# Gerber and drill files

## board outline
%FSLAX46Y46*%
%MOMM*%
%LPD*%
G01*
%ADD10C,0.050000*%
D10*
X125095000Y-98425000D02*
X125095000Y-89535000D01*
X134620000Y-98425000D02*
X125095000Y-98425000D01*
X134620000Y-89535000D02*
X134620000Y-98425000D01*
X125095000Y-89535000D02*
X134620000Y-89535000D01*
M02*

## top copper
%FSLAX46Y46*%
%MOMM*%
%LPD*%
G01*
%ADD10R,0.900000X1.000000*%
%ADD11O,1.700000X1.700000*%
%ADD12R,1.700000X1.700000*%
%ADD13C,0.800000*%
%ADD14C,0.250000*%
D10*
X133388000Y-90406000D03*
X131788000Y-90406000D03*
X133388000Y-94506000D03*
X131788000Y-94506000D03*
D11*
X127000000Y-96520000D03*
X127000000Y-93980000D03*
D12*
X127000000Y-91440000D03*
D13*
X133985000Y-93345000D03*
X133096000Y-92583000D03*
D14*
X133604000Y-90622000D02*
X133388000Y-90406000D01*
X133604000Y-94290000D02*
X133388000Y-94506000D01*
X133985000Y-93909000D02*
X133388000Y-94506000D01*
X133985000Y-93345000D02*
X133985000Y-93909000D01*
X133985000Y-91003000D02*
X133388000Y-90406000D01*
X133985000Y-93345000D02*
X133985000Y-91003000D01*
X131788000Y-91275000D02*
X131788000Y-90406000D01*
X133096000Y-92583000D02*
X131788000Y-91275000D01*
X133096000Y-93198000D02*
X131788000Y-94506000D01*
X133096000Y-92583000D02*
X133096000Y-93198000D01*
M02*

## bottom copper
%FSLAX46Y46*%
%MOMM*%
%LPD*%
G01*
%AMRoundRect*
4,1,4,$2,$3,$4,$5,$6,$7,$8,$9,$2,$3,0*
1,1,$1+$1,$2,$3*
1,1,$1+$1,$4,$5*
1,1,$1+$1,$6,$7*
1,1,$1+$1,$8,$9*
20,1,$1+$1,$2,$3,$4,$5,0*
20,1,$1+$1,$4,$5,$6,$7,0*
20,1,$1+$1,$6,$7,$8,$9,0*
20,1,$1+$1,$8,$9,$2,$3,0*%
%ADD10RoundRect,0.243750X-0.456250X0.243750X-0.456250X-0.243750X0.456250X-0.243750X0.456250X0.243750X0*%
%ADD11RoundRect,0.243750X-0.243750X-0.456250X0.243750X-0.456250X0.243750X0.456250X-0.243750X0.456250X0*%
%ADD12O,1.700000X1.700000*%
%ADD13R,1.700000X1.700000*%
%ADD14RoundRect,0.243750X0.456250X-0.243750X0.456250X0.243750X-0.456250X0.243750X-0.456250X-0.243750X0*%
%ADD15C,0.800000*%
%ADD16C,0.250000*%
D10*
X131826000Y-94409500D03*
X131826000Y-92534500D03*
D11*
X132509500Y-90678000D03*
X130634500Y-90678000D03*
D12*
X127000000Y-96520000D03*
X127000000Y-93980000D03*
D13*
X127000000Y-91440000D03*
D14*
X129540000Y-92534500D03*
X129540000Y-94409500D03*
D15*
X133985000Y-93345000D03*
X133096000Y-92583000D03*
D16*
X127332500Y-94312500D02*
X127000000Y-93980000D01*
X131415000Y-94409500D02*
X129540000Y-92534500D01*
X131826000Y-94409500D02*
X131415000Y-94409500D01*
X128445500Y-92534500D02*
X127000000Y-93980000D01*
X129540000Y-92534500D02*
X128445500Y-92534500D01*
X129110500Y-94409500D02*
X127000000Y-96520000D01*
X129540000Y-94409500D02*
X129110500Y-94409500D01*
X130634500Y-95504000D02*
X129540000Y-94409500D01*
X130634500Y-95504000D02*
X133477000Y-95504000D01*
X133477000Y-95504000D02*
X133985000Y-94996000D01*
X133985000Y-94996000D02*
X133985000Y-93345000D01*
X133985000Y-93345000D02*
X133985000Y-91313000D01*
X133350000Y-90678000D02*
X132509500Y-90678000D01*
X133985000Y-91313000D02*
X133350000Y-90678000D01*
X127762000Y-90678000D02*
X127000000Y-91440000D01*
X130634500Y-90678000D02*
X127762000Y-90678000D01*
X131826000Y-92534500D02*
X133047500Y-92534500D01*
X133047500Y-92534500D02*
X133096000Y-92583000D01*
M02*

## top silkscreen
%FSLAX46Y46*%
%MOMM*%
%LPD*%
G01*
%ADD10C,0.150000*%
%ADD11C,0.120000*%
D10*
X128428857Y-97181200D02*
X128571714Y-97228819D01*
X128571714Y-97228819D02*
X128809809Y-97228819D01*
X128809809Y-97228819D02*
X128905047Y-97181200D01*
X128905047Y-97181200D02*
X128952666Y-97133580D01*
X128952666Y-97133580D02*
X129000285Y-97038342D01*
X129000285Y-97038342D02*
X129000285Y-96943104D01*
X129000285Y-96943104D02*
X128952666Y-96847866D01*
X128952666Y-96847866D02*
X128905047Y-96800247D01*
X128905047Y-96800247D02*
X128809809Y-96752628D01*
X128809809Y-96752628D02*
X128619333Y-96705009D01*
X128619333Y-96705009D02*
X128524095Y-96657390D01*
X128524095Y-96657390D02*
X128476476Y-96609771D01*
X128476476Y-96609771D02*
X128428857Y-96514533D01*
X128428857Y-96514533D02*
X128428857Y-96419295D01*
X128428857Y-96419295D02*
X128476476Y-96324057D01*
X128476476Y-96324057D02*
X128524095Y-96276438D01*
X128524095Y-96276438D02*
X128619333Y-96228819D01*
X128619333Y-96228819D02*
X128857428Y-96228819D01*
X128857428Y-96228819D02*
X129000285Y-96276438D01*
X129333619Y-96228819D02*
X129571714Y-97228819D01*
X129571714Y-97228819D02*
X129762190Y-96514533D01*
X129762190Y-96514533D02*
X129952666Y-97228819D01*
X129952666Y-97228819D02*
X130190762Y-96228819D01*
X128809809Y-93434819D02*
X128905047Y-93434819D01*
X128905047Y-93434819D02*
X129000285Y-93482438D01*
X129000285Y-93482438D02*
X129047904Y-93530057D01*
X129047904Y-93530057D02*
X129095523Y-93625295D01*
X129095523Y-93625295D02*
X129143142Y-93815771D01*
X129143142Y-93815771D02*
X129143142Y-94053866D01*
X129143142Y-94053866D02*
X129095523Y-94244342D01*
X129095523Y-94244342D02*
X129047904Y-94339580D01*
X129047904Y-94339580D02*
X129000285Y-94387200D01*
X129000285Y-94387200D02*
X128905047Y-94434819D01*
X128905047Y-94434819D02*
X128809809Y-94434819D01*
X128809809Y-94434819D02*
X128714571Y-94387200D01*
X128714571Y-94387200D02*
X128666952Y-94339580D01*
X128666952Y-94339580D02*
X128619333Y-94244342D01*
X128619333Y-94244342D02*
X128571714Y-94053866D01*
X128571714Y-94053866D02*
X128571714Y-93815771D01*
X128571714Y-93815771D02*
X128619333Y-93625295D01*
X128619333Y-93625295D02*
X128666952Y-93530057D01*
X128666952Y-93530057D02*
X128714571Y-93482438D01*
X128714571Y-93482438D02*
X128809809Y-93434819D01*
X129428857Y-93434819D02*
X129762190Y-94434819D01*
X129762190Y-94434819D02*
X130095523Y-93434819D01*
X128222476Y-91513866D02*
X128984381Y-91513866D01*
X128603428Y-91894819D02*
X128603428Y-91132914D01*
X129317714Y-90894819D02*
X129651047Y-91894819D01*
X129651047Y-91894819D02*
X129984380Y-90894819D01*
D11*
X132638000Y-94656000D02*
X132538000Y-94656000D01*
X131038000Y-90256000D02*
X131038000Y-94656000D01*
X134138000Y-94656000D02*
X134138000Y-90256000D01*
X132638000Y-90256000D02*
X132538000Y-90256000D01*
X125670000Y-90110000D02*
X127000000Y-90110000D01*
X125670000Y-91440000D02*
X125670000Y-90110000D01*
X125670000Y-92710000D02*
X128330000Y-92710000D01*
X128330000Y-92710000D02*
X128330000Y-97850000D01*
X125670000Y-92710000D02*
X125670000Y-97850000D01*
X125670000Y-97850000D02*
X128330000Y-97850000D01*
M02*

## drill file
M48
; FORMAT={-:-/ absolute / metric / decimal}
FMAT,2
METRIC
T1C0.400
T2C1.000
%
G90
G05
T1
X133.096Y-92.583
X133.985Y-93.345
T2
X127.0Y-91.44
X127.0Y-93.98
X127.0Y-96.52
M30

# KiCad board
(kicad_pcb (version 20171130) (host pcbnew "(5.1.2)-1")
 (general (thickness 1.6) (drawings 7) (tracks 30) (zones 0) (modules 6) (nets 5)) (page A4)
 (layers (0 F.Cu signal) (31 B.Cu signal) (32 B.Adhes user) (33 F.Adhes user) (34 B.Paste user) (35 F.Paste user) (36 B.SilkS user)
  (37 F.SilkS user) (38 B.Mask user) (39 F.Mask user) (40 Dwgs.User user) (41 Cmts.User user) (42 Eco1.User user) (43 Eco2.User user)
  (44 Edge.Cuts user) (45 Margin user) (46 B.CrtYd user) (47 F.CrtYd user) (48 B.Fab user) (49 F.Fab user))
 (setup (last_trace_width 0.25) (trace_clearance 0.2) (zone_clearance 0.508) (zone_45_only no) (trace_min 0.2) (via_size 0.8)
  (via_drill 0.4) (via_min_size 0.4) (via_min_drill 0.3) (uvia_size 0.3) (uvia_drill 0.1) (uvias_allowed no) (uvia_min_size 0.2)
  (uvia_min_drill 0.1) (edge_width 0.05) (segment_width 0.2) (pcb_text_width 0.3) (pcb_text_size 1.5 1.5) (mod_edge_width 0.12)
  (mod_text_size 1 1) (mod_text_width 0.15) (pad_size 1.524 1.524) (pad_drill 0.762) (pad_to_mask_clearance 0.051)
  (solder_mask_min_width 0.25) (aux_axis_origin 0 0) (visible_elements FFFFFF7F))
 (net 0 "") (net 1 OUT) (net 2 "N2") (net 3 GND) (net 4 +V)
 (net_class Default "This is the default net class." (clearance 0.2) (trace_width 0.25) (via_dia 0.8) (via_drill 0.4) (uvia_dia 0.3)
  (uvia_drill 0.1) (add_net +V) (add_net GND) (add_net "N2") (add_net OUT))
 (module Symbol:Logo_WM (layer B.Cu) (at 131.953 97.155)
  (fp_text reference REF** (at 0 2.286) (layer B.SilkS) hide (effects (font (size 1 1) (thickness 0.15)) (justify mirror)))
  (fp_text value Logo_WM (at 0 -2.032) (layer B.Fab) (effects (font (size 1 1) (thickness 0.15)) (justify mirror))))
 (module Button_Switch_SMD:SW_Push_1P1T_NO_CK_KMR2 (layer F.Cu) (at 132.588 92.456 90)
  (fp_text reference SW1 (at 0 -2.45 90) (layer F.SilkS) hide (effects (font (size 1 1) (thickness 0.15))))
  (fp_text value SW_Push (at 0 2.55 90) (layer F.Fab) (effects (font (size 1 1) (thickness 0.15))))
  (fp_line (start -2.2 0.05) (end -2.2 -0.05) (layer F.SilkS) (width 0.12))
  (fp_line (start 2.2 -1.55) (end -2.2 -1.55) (layer F.SilkS) (width 0.12))
  (fp_line (start -2.2 1.55) (end 2.2 1.55) (layer F.SilkS) (width 0.12))
  (fp_line (start 2.2 0.05) (end 2.2 -0.05) (layer F.SilkS) (width 0.12))
  (pad 2 smd rect (at 2.05 0.8 180) (size 0.9 1) (layers F.Cu F.Paste F.Mask) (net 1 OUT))
  (pad 1 smd rect (at 2.05 -0.8 180) (size 0.9 1) (layers F.Cu F.Paste F.Mask) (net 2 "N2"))
  (pad 2 smd rect (at -2.05 0.8 180) (size 0.9 1) (layers F.Cu F.Paste F.Mask) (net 1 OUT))
  (pad 1 smd rect (at -2.05 -0.8 180) (size 0.9 1) (layers F.Cu F.Paste F.Mask) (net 2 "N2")))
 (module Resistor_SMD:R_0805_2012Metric (layer B.Cu) (at 131.826 93.472 270)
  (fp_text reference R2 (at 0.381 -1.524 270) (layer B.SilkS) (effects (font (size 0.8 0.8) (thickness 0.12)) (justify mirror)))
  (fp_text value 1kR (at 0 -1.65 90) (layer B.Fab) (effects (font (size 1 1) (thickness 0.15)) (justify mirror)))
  (pad 2 smd roundrect (at 0.9375 0 270) (size 0.975 1.4) (layers B.Cu B.Paste B.Mask) (roundrect_rratio 0.25) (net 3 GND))
  (pad 1 smd roundrect (at -0.9375 0 270) (size 0.975 1.4) (layers B.Cu B.Paste B.Mask) (roundrect_rratio 0.25) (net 2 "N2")))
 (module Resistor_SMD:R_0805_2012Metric (layer B.Cu) (at 131.572 90.678)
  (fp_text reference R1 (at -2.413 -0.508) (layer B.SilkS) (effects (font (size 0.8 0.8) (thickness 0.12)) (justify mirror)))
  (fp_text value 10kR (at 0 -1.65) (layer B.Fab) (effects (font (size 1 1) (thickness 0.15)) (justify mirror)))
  (pad 2 smd roundrect (at 0.9375 0) (size 0.975 1.4) (layers B.Cu B.Paste B.Mask) (roundrect_rratio 0.25) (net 1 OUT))
  (pad 1 smd roundrect (at -0.9375 0) (size 0.975 1.4) (layers B.Cu B.Paste B.Mask) (roundrect_rratio 0.25) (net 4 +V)))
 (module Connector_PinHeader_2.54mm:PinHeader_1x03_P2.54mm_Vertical (layer F.Cu) (at 127 91.44)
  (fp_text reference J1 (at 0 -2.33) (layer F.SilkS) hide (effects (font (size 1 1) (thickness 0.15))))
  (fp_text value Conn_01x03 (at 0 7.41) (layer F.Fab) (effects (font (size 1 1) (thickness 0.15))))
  (fp_line (start -1.33 -1.33) (end 0 -1.33) (layer F.SilkS) (width 0.12))
  (fp_line (start -1.33 0) (end -1.33 -1.33) (layer F.SilkS) (width 0.12))
  (fp_line (start -1.33 1.27) (end 1.33 1.27) (layer F.SilkS) (width 0.12))
  (fp_line (start 1.33 1.27) (end 1.33 6.41) (layer F.SilkS) (width 0.12))
  (fp_line (start -1.33 1.27) (end -1.33 6.41) (layer F.SilkS) (width 0.12))
  (fp_line (start -1.33 6.41) (end 1.33 6.41) (layer F.SilkS) (width 0.12))
  (pad 3 thru_hole oval (at 0 5.08) (size 1.7 1.7) (drill 1) (layers *.Cu *.Mask) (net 1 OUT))
  (pad 2 thru_hole oval (at 0 2.54) (size 1.7 1.7) (drill 1) (layers *.Cu *.Mask) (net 3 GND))
  (pad 1 thru_hole rect (at 0 0) (size 1.7 1.7) (drill 1) (layers *.Cu *.Mask) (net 4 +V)))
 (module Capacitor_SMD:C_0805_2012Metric (layer B.Cu) (at 129.54 93.472 90)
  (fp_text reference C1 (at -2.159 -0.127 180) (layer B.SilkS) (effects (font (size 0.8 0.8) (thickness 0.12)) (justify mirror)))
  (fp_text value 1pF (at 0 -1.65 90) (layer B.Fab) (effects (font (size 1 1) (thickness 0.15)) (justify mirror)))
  (pad 2 smd roundrect (at 0.9375 0 90) (size 0.975 1.4) (layers B.Cu B.Paste B.Mask) (roundrect_rratio 0.25) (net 3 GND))
  (pad 1 smd roundrect (at -0.9375 0 90) (size 0.975 1.4) (layers B.Cu B.Paste B.Mask) (roundrect_rratio 0.25) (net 1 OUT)))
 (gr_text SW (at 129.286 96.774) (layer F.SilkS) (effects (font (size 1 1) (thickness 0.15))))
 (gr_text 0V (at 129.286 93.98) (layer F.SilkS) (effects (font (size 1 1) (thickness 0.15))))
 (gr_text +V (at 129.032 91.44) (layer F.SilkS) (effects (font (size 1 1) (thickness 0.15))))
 (gr_line (start 125.095 98.425) (end 125.095 89.535) (layer Edge.Cuts) (width 0.05))
 (gr_line (start 134.62 98.425) (end 125.095 98.425) (layer Edge.Cuts) (width 0.05))
 (gr_line (start 134.62 89.535) (end 134.62 98.425) (layer Edge.Cuts) (width 0.05))
 (gr_line (start 125.095 89.535) (end 134.62 89.535) (layer Edge.Cuts) (width 0.05))
 (segment (start 127.3325 94.3125) (end 127 93.98) (width 0.25) (layer B.Cu) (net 3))
 (segment (start 131.415 94.4095) (end 129.54 92.5345) (width 0.25) (layer B.Cu) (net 3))
 (segment (start 131.826 94.4095) (end 131.415 94.4095) (width 0.25) (layer B.Cu) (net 3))
 (segment (start 128.4455 92.5345) (end 127 93.98) (width 0.25) (layer B.Cu) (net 3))
 (segment (start 129.54 92.5345) (end 128.4455 92.5345) (width 0.25) (layer B.Cu) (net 3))
 (segment (start 133.604 90.622) (end 133.388 90.406) (width 0.25) (layer F.Cu) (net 1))
 (segment (start 133.604 94.29) (end 133.388 94.506) (width 0.25) (layer F.Cu) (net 1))
 (segment (start 129.1105 94.4095) (end 127 96.52) (width 0.25) (layer B.Cu) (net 1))
 (segment (start 129.54 94.4095) (end 129.1105 94.4095) (width 0.25) (layer B.Cu) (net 1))
 (segment (start 130.6345 95.504) (end 129.54 94.4095) (width 0.25) (layer B.Cu) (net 1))
 (segment (start 130.6345 95.504) (end 133.477 95.504) (width 0.25) (layer B.Cu) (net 1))
 (via (at 133.985 93.345) (size 0.8) (drill 0.4) (layers F.Cu B.Cu) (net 1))
 (segment (start 133.477 95.504) (end 133.985 94.996) (width 0.25) (layer B.Cu) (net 1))
 (segment (start 133.985 94.996) (end 133.985 93.345) (width 0.25) (layer B.Cu) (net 1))
 (segment (start 133.985 93.909) (end 133.388 94.506) (width 0.25) (layer F.Cu) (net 1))
 (segment (start 133.985 93.345) (end 133.985 93.909) (width 0.25) (layer F.Cu) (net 1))
 (segment (start 133.985 91.003) (end 133.388 90.406) (width 0.25) (layer F.Cu) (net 1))
 (segment (start 133.985 93.345) (end 133.985 91.003) (width 0.25) (layer F.Cu) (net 1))
 (segment (start 133.985 93.345) (end 133.985 91.313) (width 0.25) (layer B.Cu) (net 1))
 (segment (start 133.35 90.678) (end 132.5095 90.678) (width 0.25) (layer B.Cu) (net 1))
 (segment (start 133.985 91.313) (end 133.35 90.678) (width 0.25) (layer B.Cu) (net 1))
 (segment (start 127.762 90.678) (end 127 91.44) (width 0.25) (layer B.Cu) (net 4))
 (segment (start 130.6345 90.678) (end 127.762 90.678) (width 0.25) (layer B.Cu) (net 4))
 (via (at 133.096 92.583) (size 0.8) (drill 0.4) (layers F.Cu B.Cu) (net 2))
 (segment (start 131.826 92.5345) (end 133.0475 92.5345) (width 0.25) (layer B.Cu) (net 2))
 (segment (start 133.0475 92.5345) (end 133.096 92.583) (width 0.25) (layer B.Cu) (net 2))
 (segment (start 131.788 91.275) (end 131.788 90.406) (width 0.25) (layer F.Cu) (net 2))
 (segment (start 133.096 92.583) (end 131.788 91.275) (width 0.25) (layer F.Cu) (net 2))
 (segment (start 133.096 93.198) (end 131.788 94.506) (width 0.25) (layer F.Cu) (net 2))
 (segment (start 133.096 92.583) (end 133.096 93.198) (width 0.25) (layer F.Cu) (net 2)))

